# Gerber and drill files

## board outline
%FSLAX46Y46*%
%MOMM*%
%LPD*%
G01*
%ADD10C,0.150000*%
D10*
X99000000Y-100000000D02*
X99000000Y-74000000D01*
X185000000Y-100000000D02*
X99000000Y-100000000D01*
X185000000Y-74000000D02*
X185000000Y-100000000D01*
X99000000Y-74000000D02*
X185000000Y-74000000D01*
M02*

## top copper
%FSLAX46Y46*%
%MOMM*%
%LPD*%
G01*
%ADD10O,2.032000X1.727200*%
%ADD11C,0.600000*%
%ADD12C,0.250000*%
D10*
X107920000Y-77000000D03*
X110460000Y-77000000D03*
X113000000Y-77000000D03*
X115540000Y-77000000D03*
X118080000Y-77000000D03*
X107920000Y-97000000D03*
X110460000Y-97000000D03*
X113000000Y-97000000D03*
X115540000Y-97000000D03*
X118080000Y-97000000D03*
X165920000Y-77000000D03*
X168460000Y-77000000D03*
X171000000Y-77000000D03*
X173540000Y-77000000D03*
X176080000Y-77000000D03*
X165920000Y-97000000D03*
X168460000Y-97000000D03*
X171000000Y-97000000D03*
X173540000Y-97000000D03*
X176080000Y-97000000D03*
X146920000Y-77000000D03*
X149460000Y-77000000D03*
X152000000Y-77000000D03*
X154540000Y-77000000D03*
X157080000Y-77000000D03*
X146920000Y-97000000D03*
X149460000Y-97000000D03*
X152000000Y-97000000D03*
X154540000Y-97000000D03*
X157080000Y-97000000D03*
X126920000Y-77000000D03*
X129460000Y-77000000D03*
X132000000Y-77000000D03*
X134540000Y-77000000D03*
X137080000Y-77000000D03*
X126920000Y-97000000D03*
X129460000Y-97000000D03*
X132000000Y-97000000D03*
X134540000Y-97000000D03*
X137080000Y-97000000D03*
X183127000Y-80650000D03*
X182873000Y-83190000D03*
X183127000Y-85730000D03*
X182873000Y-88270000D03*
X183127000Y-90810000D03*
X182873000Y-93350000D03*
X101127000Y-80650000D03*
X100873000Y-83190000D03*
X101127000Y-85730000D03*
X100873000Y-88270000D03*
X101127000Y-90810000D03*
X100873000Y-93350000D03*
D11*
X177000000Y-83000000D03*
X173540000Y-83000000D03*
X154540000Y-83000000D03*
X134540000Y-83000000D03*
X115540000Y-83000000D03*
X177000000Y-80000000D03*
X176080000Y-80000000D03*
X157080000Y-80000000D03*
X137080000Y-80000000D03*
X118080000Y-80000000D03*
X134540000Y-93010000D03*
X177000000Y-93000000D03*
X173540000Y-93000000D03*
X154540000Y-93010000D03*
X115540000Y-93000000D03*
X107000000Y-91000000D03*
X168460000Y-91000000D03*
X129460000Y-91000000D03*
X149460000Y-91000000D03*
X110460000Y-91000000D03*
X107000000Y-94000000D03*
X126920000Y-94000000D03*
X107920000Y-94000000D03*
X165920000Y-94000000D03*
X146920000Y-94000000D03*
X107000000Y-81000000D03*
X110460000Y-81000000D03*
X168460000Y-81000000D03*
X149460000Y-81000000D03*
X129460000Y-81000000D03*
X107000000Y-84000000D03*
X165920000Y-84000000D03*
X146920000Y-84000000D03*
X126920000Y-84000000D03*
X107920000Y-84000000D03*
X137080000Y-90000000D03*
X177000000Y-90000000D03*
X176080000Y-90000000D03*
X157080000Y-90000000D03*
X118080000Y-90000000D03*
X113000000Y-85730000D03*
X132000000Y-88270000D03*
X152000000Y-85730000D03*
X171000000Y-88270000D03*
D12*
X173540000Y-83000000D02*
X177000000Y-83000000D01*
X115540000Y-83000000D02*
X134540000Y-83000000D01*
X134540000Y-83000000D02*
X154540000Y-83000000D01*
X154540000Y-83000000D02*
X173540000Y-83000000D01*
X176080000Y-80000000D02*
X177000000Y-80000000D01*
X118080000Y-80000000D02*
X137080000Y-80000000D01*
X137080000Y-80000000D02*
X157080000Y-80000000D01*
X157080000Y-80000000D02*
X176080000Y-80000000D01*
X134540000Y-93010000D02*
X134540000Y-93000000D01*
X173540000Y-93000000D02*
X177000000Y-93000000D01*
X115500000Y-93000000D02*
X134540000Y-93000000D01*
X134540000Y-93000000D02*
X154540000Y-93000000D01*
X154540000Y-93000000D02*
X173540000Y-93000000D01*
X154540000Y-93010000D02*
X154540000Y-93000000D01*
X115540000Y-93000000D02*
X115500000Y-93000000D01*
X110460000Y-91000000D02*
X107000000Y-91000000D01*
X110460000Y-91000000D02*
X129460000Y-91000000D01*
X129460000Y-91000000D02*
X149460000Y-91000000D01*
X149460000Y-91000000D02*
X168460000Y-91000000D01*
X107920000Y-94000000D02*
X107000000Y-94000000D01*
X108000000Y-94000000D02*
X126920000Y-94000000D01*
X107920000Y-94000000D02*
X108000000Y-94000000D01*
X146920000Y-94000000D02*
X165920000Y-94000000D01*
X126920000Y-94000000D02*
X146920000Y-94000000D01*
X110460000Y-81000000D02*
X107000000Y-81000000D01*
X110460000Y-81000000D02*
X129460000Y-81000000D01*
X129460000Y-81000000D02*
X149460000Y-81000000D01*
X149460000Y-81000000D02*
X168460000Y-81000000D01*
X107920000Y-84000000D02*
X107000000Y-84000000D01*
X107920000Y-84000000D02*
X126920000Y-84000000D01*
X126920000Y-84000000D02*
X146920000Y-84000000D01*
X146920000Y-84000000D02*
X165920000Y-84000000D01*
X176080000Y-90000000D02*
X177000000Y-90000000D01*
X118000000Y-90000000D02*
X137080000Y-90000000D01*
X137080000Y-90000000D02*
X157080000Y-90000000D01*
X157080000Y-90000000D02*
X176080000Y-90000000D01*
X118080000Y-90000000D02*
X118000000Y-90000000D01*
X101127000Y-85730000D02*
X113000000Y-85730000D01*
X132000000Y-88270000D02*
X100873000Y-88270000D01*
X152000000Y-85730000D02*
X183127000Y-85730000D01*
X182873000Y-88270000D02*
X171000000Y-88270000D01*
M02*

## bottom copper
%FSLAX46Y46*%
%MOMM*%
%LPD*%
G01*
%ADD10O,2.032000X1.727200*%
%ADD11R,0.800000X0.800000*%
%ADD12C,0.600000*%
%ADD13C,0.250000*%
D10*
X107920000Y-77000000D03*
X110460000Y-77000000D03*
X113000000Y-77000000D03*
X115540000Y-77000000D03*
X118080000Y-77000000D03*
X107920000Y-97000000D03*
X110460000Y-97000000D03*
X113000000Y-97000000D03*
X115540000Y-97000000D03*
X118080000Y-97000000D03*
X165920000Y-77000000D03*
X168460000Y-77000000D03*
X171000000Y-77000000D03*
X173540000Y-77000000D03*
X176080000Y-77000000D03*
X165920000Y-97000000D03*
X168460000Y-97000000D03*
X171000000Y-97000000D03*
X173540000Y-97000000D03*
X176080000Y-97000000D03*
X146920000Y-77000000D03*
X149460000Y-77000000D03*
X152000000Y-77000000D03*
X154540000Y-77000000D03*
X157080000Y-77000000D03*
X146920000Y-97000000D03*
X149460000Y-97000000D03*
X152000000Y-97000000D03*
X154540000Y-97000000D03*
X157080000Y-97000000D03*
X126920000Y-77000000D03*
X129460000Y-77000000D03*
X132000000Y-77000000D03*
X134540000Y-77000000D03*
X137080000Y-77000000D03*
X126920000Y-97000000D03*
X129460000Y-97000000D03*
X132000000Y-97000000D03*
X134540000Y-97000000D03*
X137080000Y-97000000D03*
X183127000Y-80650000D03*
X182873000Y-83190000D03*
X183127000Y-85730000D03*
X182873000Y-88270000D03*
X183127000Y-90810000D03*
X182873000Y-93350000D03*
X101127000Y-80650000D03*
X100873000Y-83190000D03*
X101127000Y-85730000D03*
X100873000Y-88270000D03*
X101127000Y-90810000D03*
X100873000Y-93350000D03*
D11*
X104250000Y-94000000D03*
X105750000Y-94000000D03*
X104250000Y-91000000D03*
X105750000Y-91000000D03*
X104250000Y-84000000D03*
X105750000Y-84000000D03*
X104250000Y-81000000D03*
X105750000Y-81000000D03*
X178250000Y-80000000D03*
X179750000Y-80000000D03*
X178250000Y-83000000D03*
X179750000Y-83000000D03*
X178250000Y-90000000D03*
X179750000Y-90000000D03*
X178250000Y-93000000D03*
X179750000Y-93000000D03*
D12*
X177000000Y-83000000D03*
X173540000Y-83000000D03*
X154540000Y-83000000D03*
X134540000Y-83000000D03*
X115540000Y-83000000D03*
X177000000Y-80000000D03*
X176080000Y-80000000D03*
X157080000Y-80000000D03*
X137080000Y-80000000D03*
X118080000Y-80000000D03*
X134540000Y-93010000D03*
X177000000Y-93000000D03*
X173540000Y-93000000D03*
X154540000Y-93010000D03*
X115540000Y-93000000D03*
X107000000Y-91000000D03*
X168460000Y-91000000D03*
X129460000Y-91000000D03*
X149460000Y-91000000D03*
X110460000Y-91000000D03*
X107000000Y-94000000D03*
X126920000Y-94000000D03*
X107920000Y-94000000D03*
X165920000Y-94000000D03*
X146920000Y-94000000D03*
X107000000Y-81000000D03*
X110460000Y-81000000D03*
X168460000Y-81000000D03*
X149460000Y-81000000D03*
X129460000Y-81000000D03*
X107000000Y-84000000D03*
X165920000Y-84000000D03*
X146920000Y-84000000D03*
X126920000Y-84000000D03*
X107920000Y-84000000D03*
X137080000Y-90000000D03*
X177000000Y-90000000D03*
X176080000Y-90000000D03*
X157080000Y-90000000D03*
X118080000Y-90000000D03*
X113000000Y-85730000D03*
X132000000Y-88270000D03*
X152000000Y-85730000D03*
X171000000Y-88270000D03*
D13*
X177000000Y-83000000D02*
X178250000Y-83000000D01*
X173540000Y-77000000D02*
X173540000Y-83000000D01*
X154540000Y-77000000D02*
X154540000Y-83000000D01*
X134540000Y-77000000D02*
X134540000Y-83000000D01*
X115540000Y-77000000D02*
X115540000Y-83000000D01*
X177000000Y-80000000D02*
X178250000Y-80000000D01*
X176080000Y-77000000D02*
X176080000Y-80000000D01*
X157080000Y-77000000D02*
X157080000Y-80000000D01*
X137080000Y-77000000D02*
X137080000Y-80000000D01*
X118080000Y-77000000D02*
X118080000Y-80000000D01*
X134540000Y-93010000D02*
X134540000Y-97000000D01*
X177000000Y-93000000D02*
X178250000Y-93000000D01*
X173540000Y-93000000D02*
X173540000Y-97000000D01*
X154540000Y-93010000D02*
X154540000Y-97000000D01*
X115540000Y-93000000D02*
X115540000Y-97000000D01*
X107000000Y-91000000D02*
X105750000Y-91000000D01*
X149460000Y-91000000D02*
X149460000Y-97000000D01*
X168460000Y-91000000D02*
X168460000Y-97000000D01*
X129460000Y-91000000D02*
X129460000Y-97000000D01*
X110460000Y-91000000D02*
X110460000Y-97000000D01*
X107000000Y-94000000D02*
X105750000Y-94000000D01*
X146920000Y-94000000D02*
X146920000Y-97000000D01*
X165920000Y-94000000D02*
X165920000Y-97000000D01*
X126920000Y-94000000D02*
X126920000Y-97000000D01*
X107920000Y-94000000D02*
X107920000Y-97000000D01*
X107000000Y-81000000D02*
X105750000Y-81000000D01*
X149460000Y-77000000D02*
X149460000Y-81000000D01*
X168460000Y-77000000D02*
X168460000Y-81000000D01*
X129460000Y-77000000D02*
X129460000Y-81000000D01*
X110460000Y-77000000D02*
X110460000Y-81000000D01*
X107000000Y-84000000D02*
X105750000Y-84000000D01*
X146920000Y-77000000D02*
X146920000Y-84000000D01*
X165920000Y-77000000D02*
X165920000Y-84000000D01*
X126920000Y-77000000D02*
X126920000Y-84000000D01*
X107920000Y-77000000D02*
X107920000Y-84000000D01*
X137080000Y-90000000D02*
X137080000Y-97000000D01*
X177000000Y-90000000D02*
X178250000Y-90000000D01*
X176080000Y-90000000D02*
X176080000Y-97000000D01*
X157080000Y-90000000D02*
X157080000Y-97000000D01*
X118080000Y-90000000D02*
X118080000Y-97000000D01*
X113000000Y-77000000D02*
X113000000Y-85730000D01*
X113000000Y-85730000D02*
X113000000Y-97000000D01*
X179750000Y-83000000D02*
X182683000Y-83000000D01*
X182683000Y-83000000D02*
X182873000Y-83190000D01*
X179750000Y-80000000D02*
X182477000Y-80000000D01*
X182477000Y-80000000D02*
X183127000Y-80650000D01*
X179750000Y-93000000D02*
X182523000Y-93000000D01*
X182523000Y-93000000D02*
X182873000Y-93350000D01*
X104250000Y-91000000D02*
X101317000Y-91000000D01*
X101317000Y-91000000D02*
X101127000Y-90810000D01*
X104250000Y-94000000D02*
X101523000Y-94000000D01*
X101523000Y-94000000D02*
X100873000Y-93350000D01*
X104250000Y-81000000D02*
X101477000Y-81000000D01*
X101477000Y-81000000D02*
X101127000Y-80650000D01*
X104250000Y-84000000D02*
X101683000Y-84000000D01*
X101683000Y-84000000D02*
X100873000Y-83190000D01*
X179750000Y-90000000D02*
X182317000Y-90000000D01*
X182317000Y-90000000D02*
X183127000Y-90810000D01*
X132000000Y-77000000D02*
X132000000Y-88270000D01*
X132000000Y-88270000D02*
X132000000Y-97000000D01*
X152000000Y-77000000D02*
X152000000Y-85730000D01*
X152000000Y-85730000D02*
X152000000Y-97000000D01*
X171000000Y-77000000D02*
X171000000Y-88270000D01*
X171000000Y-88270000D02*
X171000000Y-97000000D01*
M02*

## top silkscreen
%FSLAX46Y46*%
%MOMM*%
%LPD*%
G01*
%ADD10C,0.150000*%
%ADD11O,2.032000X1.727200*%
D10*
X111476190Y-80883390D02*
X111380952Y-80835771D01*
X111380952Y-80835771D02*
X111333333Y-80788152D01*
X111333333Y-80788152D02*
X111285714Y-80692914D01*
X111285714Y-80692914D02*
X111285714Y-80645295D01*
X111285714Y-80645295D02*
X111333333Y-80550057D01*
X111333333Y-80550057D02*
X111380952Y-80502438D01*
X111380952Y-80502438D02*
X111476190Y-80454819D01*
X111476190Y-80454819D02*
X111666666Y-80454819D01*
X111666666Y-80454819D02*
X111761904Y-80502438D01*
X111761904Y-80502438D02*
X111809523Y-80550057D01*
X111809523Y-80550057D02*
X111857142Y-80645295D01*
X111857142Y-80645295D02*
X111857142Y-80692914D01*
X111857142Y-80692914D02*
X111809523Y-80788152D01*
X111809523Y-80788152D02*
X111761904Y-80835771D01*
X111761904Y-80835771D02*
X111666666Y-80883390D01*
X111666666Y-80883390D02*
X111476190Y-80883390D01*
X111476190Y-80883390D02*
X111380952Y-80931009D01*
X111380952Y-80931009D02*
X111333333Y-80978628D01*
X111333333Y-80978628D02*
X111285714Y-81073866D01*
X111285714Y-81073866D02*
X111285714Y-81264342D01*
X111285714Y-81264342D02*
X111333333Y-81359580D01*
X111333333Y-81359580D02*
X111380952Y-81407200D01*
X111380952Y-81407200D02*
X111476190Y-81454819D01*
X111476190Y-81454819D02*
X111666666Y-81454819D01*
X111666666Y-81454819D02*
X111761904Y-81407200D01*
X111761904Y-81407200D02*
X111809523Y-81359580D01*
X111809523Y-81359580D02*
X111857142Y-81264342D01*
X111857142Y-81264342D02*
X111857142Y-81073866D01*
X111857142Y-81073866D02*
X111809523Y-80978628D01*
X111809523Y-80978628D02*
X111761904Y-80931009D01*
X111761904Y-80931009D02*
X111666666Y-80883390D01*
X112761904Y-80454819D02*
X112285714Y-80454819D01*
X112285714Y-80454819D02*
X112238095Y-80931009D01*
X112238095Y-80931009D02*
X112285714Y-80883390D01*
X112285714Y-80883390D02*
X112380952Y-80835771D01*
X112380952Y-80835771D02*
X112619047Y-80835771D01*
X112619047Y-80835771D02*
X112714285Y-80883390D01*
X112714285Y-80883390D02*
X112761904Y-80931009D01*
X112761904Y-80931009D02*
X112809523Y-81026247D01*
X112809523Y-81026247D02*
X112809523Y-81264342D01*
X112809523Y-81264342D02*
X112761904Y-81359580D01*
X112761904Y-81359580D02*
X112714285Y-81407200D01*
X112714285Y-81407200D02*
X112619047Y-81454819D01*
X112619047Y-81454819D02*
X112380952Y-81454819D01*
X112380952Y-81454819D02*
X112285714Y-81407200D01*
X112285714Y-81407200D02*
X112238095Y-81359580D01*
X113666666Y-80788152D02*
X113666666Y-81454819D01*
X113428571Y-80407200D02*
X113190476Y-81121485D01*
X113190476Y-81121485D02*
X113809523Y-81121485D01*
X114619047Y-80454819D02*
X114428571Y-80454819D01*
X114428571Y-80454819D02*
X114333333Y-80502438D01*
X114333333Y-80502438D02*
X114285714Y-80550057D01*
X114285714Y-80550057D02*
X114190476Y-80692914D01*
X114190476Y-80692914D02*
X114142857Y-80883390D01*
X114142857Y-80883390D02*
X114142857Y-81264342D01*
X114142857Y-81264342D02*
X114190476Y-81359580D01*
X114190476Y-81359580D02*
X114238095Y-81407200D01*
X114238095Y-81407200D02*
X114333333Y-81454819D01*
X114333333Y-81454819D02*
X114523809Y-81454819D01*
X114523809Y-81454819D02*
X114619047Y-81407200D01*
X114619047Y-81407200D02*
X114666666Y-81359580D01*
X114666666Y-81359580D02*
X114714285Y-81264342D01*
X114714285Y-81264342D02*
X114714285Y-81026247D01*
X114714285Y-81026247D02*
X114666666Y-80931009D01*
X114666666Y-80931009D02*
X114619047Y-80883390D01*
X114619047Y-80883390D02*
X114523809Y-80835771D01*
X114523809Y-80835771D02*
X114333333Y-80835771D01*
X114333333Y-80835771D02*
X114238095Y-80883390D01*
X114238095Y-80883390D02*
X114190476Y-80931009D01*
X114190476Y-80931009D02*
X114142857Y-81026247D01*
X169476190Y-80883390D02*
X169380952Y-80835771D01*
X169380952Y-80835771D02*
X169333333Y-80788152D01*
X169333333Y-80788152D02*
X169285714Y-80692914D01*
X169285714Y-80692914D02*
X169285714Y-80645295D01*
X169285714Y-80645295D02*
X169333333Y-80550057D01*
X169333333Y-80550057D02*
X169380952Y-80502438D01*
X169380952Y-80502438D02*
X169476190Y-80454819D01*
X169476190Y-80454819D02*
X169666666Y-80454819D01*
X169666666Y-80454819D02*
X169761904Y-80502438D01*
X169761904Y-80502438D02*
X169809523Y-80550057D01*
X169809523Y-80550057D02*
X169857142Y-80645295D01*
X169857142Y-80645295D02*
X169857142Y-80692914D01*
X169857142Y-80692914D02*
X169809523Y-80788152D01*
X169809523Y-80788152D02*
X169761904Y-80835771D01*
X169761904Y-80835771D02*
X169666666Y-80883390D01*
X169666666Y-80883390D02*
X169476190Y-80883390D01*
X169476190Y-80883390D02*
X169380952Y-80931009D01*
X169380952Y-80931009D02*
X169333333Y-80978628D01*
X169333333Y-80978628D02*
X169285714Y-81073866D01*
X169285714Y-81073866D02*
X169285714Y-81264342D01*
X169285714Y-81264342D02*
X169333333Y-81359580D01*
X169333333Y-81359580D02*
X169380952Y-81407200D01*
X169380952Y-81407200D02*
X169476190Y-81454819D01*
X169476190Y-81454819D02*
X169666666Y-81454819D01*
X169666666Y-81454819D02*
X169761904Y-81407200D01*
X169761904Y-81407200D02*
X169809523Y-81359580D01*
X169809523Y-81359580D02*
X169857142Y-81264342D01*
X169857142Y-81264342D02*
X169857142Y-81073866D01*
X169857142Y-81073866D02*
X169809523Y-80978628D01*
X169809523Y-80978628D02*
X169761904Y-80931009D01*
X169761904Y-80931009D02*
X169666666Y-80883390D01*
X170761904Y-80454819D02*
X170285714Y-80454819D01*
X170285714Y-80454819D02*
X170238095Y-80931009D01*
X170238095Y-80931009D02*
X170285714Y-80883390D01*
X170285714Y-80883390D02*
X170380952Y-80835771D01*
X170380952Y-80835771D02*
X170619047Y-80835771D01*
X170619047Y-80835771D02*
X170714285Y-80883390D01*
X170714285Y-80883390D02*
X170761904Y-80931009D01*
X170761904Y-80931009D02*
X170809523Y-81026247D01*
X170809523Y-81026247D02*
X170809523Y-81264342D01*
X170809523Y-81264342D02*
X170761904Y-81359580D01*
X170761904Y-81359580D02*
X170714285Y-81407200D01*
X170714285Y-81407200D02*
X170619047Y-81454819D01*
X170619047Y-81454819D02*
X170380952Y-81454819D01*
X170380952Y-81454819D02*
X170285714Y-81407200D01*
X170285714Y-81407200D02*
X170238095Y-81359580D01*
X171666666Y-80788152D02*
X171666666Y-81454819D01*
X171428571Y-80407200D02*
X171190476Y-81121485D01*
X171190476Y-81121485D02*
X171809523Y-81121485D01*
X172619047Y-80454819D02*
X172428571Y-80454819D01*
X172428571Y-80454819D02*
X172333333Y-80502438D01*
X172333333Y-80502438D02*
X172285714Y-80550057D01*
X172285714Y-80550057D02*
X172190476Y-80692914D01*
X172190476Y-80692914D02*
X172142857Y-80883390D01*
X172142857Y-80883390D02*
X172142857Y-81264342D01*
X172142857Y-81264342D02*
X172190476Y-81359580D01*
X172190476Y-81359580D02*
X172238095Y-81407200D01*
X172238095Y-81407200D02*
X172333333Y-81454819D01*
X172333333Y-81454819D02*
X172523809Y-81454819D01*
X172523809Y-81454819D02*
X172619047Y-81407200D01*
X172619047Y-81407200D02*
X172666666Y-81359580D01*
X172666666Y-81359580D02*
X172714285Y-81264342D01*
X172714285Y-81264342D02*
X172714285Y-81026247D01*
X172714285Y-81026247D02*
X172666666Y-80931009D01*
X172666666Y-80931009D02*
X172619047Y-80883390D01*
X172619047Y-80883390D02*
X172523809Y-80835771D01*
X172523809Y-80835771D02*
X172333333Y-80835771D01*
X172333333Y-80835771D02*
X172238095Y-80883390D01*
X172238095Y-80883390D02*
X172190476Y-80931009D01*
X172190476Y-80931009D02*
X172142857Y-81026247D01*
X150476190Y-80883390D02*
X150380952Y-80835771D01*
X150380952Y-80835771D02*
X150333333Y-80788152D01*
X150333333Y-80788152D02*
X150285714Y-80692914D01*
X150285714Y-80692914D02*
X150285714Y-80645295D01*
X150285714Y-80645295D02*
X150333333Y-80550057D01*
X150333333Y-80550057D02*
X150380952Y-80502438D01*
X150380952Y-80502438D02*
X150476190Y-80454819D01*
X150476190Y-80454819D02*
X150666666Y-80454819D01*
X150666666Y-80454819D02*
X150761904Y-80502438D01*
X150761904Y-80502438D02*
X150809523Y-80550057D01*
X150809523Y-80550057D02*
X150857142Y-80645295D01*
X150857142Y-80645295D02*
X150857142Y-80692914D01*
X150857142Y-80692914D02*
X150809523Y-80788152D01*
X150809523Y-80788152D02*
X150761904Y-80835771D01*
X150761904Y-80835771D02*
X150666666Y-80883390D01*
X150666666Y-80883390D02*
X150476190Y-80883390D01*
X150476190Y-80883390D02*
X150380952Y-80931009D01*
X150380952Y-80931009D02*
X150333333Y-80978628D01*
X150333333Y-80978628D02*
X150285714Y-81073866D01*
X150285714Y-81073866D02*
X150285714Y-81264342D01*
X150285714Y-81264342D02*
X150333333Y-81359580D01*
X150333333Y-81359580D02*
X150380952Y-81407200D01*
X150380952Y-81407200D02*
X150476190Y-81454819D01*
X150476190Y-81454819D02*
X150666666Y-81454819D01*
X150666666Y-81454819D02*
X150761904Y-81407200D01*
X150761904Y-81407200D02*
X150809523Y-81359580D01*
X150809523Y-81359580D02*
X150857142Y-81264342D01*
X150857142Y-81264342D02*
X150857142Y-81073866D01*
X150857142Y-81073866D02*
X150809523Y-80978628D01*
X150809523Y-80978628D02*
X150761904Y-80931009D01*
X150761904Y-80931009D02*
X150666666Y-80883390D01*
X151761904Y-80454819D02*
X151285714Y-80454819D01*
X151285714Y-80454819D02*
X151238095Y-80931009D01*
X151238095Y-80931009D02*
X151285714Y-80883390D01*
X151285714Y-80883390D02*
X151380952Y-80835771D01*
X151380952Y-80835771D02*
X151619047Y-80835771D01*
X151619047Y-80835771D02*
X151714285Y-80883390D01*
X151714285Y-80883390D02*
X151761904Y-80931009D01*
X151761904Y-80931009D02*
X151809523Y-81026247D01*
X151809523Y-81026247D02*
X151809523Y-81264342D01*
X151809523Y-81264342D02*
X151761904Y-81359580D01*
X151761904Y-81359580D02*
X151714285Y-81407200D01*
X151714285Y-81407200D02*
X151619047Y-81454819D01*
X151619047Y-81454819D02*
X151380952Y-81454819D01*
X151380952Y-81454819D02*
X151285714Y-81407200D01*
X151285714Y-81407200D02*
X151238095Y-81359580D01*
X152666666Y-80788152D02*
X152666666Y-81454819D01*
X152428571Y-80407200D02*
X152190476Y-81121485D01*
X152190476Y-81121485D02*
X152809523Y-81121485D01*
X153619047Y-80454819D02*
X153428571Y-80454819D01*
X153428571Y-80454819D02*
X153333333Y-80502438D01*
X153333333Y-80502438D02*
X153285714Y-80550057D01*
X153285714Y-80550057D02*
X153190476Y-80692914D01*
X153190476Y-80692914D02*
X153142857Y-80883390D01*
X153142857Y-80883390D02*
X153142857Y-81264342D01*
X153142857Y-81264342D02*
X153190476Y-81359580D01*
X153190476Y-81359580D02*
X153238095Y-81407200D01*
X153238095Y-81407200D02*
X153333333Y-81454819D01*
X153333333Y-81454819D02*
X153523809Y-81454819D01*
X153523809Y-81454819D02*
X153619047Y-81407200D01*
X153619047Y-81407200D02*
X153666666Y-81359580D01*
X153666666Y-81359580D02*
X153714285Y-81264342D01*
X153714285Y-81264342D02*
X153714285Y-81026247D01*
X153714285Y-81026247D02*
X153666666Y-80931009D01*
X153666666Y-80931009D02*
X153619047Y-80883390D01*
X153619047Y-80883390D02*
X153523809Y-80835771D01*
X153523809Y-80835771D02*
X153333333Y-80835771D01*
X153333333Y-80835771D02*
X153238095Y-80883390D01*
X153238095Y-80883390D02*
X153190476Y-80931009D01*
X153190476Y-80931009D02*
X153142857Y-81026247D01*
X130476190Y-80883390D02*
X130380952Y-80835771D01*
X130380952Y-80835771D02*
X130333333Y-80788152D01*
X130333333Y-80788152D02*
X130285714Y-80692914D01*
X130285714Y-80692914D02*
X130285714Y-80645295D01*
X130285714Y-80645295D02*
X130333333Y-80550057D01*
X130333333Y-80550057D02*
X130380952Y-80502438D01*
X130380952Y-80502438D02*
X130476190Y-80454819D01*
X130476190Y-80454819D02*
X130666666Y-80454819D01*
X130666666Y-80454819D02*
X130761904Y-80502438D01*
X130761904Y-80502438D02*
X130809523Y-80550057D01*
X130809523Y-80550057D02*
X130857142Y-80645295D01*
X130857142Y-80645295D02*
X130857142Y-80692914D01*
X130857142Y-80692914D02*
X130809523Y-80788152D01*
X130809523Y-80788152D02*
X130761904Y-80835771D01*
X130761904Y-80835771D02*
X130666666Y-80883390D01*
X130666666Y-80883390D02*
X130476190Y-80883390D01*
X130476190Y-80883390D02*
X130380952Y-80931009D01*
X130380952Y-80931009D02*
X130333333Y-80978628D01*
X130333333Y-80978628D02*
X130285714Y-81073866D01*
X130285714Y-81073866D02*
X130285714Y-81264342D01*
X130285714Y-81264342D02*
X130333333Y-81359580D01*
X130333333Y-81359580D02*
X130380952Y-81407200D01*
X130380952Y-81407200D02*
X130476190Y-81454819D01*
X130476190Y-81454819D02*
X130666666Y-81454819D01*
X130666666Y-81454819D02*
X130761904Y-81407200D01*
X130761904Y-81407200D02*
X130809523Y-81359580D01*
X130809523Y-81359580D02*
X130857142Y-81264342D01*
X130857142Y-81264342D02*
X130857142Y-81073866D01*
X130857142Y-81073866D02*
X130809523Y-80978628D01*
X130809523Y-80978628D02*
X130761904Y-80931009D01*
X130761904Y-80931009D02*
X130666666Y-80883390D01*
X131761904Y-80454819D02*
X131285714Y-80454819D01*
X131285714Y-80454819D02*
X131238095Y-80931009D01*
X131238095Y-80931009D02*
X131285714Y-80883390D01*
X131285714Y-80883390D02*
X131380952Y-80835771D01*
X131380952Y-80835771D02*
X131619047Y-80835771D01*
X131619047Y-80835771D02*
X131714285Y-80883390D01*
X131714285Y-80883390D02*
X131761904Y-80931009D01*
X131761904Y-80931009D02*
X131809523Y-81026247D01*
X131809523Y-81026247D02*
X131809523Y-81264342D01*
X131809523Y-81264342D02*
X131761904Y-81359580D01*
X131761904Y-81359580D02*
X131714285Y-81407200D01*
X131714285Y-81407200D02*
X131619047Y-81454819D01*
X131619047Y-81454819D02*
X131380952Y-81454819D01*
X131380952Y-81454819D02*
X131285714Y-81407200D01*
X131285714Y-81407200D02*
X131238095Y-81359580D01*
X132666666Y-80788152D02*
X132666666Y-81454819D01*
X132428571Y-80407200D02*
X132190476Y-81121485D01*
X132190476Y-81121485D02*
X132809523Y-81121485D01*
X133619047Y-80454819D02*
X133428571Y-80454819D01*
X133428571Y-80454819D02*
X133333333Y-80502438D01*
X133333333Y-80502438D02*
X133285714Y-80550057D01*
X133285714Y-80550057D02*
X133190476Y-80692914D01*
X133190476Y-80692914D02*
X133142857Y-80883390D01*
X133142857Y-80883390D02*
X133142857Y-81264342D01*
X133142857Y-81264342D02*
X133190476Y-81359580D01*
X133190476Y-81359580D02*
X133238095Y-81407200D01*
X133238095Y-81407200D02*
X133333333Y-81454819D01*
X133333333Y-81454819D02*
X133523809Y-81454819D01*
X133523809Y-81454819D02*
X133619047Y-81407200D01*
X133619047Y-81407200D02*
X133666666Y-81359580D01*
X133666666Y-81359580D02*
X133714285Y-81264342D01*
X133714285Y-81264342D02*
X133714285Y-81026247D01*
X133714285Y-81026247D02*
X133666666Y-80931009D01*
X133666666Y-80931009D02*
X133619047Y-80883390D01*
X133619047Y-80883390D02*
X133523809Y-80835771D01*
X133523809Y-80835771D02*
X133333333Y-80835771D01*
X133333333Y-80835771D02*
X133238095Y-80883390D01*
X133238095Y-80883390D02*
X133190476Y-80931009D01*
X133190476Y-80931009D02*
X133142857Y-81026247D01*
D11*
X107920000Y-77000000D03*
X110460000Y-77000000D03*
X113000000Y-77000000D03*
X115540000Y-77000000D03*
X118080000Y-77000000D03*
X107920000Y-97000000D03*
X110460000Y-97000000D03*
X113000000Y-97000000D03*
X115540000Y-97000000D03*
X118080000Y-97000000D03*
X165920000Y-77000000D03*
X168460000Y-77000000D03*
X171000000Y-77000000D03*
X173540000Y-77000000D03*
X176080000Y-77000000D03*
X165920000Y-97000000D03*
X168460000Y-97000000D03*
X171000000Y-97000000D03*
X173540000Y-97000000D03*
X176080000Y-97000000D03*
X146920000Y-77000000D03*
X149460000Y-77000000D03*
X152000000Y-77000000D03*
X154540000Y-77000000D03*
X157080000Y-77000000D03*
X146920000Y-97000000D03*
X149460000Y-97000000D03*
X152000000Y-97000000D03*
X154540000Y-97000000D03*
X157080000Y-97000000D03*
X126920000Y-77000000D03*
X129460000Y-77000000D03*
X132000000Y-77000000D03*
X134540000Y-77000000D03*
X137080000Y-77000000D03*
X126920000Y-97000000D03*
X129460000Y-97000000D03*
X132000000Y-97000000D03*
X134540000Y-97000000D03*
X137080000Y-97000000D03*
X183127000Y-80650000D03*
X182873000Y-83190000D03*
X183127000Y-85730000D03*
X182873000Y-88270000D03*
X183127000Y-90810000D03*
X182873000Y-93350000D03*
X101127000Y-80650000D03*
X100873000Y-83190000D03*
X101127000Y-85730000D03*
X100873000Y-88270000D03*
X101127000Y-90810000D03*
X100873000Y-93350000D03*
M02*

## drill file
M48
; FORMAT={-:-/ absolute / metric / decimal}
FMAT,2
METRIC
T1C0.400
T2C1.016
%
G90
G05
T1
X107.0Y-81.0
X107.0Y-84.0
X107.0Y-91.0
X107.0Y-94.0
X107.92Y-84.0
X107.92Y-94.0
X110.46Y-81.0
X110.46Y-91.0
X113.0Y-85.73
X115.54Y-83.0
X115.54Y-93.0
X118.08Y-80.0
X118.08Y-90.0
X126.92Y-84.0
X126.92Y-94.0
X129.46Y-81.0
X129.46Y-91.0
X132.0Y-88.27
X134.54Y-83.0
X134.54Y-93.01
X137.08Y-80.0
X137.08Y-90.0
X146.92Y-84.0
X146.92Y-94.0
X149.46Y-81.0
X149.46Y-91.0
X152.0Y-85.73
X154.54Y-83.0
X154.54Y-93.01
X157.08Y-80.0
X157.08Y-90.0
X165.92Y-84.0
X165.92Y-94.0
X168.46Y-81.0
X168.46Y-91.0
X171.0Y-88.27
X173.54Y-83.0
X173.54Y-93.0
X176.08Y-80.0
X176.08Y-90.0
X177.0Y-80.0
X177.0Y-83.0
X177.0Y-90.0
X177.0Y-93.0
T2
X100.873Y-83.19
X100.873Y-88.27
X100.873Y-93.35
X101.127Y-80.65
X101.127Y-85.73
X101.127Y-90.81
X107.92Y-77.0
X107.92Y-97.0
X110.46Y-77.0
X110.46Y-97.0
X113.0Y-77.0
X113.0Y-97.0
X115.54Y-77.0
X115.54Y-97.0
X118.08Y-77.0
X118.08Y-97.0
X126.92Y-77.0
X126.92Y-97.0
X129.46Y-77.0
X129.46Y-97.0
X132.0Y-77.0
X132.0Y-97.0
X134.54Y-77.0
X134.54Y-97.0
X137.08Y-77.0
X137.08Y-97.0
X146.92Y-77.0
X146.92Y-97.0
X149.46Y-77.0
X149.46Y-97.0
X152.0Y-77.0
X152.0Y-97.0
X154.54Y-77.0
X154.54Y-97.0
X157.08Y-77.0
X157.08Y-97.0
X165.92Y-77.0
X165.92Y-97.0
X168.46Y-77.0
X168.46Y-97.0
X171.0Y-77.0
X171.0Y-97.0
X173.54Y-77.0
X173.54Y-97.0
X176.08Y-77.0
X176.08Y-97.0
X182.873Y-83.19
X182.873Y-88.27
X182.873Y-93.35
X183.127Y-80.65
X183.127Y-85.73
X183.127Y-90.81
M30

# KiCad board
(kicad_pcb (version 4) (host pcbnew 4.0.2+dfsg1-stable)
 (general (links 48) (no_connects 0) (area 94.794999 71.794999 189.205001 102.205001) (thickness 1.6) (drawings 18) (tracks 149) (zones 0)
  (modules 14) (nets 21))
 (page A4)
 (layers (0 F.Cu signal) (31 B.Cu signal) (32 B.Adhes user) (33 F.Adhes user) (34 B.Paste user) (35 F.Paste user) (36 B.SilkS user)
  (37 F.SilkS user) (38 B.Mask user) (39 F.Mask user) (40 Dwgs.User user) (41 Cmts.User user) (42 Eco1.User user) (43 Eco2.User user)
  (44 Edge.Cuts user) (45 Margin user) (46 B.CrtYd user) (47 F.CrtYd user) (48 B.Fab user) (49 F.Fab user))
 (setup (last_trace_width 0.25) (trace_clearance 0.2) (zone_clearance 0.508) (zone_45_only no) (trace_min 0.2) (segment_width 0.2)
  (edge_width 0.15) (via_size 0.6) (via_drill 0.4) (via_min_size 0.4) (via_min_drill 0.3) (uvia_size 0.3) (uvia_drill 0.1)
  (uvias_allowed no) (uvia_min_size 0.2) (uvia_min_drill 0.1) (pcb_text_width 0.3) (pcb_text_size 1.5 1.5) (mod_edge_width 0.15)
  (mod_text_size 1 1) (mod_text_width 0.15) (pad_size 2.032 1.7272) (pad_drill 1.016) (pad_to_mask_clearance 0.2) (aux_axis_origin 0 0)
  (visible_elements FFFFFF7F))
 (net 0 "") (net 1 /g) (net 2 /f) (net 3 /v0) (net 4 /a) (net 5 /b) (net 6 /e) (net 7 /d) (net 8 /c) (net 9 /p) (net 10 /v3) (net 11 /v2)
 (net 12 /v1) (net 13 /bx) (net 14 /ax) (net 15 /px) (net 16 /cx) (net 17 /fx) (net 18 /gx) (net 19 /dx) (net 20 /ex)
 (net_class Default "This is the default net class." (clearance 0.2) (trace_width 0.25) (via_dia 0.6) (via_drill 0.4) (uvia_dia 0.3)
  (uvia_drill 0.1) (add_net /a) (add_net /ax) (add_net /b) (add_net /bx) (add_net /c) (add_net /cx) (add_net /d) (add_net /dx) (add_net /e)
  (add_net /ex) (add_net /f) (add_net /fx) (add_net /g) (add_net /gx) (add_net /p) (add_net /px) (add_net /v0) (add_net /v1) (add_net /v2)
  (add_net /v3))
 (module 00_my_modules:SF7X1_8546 (layer F.Cu) (at 113 87)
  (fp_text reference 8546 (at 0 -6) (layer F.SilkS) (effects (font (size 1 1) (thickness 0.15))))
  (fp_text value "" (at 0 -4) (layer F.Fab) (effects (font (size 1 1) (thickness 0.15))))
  (pad G thru_hole oval (at -5.08 -10) (size 2.032 1.7272) (drill 1.016) (layers *.Cu *.Mask F.SilkS) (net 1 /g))
  (pad F thru_hole oval (at -2.54 -10) (size 2.032 1.7272) (drill 1.016) (layers *.Cu *.Mask F.SilkS) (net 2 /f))
  (pad V thru_hole oval (at 0 -10) (size 2.032 1.7272) (drill 1.016) (layers *.Cu *.Mask F.SilkS) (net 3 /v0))
  (pad A thru_hole oval (at 2.54 -10) (size 2.032 1.7272) (drill 1.016) (layers *.Cu *.Mask F.SilkS) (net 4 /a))
  (pad B thru_hole oval (at 5.08 -10) (size 2.032 1.7272) (drill 1.016) (layers *.Cu *.Mask F.SilkS) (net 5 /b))
  (pad E thru_hole oval (at -5.08 10) (size 2.032 1.7272) (drill 1.016) (layers *.Cu *.Mask F.SilkS) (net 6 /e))
  (pad D thru_hole oval (at -2.54 10) (size 2.032 1.7272) (drill 1.016) (layers *.Cu *.Mask F.SilkS) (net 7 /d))
  (pad V thru_hole oval (at 0 10) (size 2.032 1.7272) (drill 1.016) (layers *.Cu *.Mask F.SilkS) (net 3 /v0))
  (pad C thru_hole oval (at 2.54 10) (size 2.032 1.7272) (drill 1.016) (layers *.Cu *.Mask F.SilkS) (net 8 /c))
  (pad P thru_hole oval (at 5.08 10) (size 2.032 1.7272) (drill 1.016) (layers *.Cu *.Mask F.SilkS) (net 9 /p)))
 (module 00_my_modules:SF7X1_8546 (layer F.Cu) (at 171 87)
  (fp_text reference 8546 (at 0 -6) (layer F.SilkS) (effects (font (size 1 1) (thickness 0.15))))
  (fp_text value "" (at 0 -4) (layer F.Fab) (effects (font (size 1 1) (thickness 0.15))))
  (pad G thru_hole oval (at -5.08 -10) (size 2.032 1.7272) (drill 1.016) (layers *.Cu *.Mask F.SilkS) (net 1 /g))
  (pad F thru_hole oval (at -2.54 -10) (size 2.032 1.7272) (drill 1.016) (layers *.Cu *.Mask F.SilkS) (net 2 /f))
  (pad V thru_hole oval (at 0 -10) (size 2.032 1.7272) (drill 1.016) (layers *.Cu *.Mask F.SilkS) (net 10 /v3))
  (pad A thru_hole oval (at 2.54 -10) (size 2.032 1.7272) (drill 1.016) (layers *.Cu *.Mask F.SilkS) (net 4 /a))
  (pad B thru_hole oval (at 5.08 -10) (size 2.032 1.7272) (drill 1.016) (layers *.Cu *.Mask F.SilkS) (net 5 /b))
  (pad E thru_hole oval (at -5.08 10) (size 2.032 1.7272) (drill 1.016) (layers *.Cu *.Mask F.SilkS) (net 6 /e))
  (pad D thru_hole oval (at -2.54 10) (size 2.032 1.7272) (drill 1.016) (layers *.Cu *.Mask F.SilkS) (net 7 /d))
  (pad V thru_hole oval (at 0 10) (size 2.032 1.7272) (drill 1.016) (layers *.Cu *.Mask F.SilkS) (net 10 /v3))
  (pad C thru_hole oval (at 2.54 10) (size 2.032 1.7272) (drill 1.016) (layers *.Cu *.Mask F.SilkS) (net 8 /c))
  (pad P thru_hole oval (at 5.08 10) (size 2.032 1.7272) (drill 1.016) (layers *.Cu *.Mask F.SilkS) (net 9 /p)))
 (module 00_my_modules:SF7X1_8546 (layer F.Cu) (at 152 87)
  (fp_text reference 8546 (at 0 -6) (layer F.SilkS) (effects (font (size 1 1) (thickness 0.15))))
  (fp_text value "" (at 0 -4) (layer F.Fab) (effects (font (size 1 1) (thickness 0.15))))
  (pad G thru_hole oval (at -5.08 -10) (size 2.032 1.7272) (drill 1.016) (layers *.Cu *.Mask F.SilkS) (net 1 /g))
  (pad F thru_hole oval (at -2.54 -10) (size 2.032 1.7272) (drill 1.016) (layers *.Cu *.Mask F.SilkS) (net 2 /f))
  (pad V thru_hole oval (at 0 -10) (size 2.032 1.7272) (drill 1.016) (layers *.Cu *.Mask F.SilkS) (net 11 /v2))
  (pad A thru_hole oval (at 2.54 -10) (size 2.032 1.7272) (drill 1.016) (layers *.Cu *.Mask F.SilkS) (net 4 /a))
  (pad B thru_hole oval (at 5.08 -10) (size 2.032 1.7272) (drill 1.016) (layers *.Cu *.Mask F.SilkS) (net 5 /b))
  (pad E thru_hole oval (at -5.08 10) (size 2.032 1.7272) (drill 1.016) (layers *.Cu *.Mask F.SilkS) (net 6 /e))
  (pad D thru_hole oval (at -2.54 10) (size 2.032 1.7272) (drill 1.016) (layers *.Cu *.Mask F.SilkS) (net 7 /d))
  (pad V thru_hole oval (at 0 10) (size 2.032 1.7272) (drill 1.016) (layers *.Cu *.Mask F.SilkS) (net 11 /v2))
  (pad C thru_hole oval (at 2.54 10) (size 2.032 1.7272) (drill 1.016) (layers *.Cu *.Mask F.SilkS) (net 8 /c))
  (pad P thru_hole oval (at 5.08 10) (size 2.032 1.7272) (drill 1.016) (layers *.Cu *.Mask F.SilkS) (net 9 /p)))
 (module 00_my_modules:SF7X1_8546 (layer F.Cu) (at 132 87)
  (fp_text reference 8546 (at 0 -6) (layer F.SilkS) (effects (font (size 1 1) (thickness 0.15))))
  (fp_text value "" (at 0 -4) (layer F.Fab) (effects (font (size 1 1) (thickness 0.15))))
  (pad G thru_hole oval (at -5.08 -10) (size 2.032 1.7272) (drill 1.016) (layers *.Cu *.Mask F.SilkS) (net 1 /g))
  (pad F thru_hole oval (at -2.54 -10) (size 2.032 1.7272) (drill 1.016) (layers *.Cu *.Mask F.SilkS) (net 2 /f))
  (pad V thru_hole oval (at 0 -10) (size 2.032 1.7272) (drill 1.016) (layers *.Cu *.Mask F.SilkS) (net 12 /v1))
  (pad A thru_hole oval (at 2.54 -10) (size 2.032 1.7272) (drill 1.016) (layers *.Cu *.Mask F.SilkS) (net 4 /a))
  (pad B thru_hole oval (at 5.08 -10) (size 2.032 1.7272) (drill 1.016) (layers *.Cu *.Mask F.SilkS) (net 5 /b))
  (pad E thru_hole oval (at -5.08 10) (size 2.032 1.7272) (drill 1.016) (layers *.Cu *.Mask F.SilkS) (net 6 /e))
  (pad D thru_hole oval (at -2.54 10) (size 2.032 1.7272) (drill 1.016) (layers *.Cu *.Mask F.SilkS) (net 7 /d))
  (pad V thru_hole oval (at 0 10) (size 2.032 1.7272) (drill 1.016) (layers *.Cu *.Mask F.SilkS) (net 12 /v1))
  (pad C thru_hole oval (at 2.54 10) (size 2.032 1.7272) (drill 1.016) (layers *.Cu *.Mask F.SilkS) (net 8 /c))
  (pad P thru_hole oval (at 5.08 10) (size 2.032 1.7272) (drill 1.016) (layers *.Cu *.Mask F.SilkS) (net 9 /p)))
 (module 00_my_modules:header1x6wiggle (layer F.Cu) (at 183 87)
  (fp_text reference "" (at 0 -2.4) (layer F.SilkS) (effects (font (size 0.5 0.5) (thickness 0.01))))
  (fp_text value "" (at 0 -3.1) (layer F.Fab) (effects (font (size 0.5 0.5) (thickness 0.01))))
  (pad 1 thru_hole oval (at 0.127 -6.35) (size 2.032 1.7272) (drill 1.016) (layers *.Cu *.Mask F.SilkS) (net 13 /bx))
  (pad 2 thru_hole oval (at -0.127 -3.81) (size 2.032 1.7272) (drill 1.016) (layers *.Cu *.Mask F.SilkS) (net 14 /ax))
  (pad 3 thru_hole oval (at 0.127 -1.27) (size 2.032 1.7272) (drill 1.016) (layers *.Cu *.Mask F.SilkS) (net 11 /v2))
  (pad 4 thru_hole oval (at -0.127 1.27) (size 2.032 1.7272) (drill 1.016) (layers *.Cu *.Mask F.SilkS) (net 10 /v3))
  (pad 5 thru_hole oval (at 0.127 3.81) (size 2.032 1.7272) (drill 1.016) (layers *.Cu *.Mask F.SilkS) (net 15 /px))
  (pad 6 thru_hole oval (at -0.127 6.35) (size 2.032 1.7272) (drill 1.016) (layers *.Cu *.Mask F.SilkS) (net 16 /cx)))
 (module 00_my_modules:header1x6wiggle (layer F.Cu) (at 101 87)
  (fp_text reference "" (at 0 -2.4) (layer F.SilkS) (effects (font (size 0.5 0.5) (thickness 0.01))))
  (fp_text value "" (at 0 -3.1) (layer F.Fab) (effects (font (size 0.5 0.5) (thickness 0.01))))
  (pad 1 thru_hole oval (at 0.127 -6.35) (size 2.032 1.7272) (drill 1.016) (layers *.Cu *.Mask F.SilkS) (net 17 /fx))
  (pad 2 thru_hole oval (at -0.127 -3.81) (size 2.032 1.7272) (drill 1.016) (layers *.Cu *.Mask F.SilkS) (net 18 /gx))
  (pad 3 thru_hole oval (at 0.127 -1.27) (size 2.032 1.7272) (drill 1.016) (layers *.Cu *.Mask F.SilkS) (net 3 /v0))
  (pad 4 thru_hole oval (at -0.127 1.27) (size 2.032 1.7272) (drill 1.016) (layers *.Cu *.Mask F.SilkS) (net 12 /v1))
  (pad 5 thru_hole oval (at 0.127 3.81) (size 2.032 1.7272) (drill 1.016) (layers *.Cu *.Mask F.SilkS) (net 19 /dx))
  (pad 6 thru_hole oval (at -0.127 6.35) (size 2.032 1.7272) (drill 1.016) (layers *.Cu *.Mask F.SilkS) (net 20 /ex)))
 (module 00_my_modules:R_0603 (layer B.Cu) (at 105 94)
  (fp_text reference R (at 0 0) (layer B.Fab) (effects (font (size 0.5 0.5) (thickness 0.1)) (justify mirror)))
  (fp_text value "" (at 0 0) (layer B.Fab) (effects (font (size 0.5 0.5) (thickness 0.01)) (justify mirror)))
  (pad 1 smd rect (at -0.75 0) (size 0.8 0.8) (layers B.Cu B.Paste B.Mask) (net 20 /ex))
  (pad 2 smd rect (at 0.75 0) (size 0.8 0.8) (layers B.Cu B.Paste B.Mask) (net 6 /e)))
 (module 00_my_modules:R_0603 (layer B.Cu) (at 105 91)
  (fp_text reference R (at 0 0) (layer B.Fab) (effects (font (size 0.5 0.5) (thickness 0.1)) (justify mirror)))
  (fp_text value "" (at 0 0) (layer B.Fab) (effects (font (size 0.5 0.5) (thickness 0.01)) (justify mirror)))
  (pad 1 smd rect (at -0.75 0) (size 0.8 0.8) (layers B.Cu B.Paste B.Mask) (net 19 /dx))
  (pad 2 smd rect (at 0.75 0) (size 0.8 0.8) (layers B.Cu B.Paste B.Mask) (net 7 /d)))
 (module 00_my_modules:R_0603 (layer B.Cu) (at 105 84)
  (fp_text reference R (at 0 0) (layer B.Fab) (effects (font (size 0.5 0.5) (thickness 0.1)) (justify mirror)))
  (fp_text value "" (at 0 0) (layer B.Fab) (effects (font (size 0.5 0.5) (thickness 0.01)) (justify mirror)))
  (pad 1 smd rect (at -0.75 0) (size 0.8 0.8) (layers B.Cu B.Paste B.Mask) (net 18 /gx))
  (pad 2 smd rect (at 0.75 0) (size 0.8 0.8) (layers B.Cu B.Paste B.Mask) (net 1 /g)))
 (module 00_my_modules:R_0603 (layer B.Cu) (at 105 81)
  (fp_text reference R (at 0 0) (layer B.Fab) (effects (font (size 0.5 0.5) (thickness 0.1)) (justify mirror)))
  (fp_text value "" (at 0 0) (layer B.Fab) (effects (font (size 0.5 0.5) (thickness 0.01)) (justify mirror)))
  (pad 1 smd rect (at -0.75 0) (size 0.8 0.8) (layers B.Cu B.Paste B.Mask) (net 17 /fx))
  (pad 2 smd rect (at 0.75 0) (size 0.8 0.8) (layers B.Cu B.Paste B.Mask) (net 2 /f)))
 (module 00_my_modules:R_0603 (layer B.Cu) (at 179 80)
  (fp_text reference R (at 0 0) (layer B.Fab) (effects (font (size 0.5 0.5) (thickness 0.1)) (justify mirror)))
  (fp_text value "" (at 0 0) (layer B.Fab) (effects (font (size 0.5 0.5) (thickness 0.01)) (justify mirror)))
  (pad 1 smd rect (at -0.75 0) (size 0.8 0.8) (layers B.Cu B.Paste B.Mask) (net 5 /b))
  (pad 2 smd rect (at 0.75 0) (size 0.8 0.8) (layers B.Cu B.Paste B.Mask) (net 13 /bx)))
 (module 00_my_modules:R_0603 (layer B.Cu) (at 179 83)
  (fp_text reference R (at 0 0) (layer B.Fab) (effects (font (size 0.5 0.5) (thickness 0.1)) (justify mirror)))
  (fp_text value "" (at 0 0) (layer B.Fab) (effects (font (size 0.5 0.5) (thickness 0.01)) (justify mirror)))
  (pad 1 smd rect (at -0.75 0) (size 0.8 0.8) (layers B.Cu B.Paste B.Mask) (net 4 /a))
  (pad 2 smd rect (at 0.75 0) (size 0.8 0.8) (layers B.Cu B.Paste B.Mask) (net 14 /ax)))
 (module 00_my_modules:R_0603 (layer B.Cu) (at 179 90)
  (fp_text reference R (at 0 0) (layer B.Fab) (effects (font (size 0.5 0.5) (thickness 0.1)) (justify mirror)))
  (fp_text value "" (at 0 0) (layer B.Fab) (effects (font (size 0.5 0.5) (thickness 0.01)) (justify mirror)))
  (pad 1 smd rect (at -0.75 0) (size 0.8 0.8) (layers B.Cu B.Paste B.Mask) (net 9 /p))
  (pad 2 smd rect (at 0.75 0) (size 0.8 0.8) (layers B.Cu B.Paste B.Mask) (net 15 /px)))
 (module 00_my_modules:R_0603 (layer B.Cu) (at 179 93)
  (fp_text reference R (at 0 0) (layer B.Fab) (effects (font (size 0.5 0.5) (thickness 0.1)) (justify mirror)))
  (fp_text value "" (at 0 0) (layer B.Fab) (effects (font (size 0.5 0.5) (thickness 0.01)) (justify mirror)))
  (pad 1 smd rect (at -0.75 0) (size 0.8 0.8) (layers B.Cu B.Paste B.Mask) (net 8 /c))
  (pad 2 smd rect (at 0.75 0) (size 0.8 0.8) (layers B.Cu B.Paste B.Mask) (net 16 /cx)))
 (gr_line (start 99 100) (end 99 74) (angle 90) (layer Edge.Cuts) (width 0.15))
 (gr_line (start 185 100) (end 99 100) (angle 90) (layer Edge.Cuts) (width 0.15))
 (gr_line (start 185 74) (end 185 100) (angle 90) (layer Edge.Cuts) (width 0.15))
 (gr_line (start 99 74) (end 185 74) (angle 90) (layer Edge.Cuts) (width 0.15))
 (segment (start 173.54 83) (end 177 83) (width 0.25) (layer F.Cu) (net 4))
 (segment (start 177 83) (end 178.25 83) (width 0.25) (layer B.Cu) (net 4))
 (via (at 177 83) (size 0.6) (drill 0.4) (layers F.Cu B.Cu) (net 4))
 (segment (start 115.54 83) (end 134.54 83) (width 0.25) (layer F.Cu) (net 4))
 (segment (start 134.54 83) (end 154.54 83) (width 0.25) (layer F.Cu) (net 4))
 (segment (start 154.54 83) (end 173.54 83) (width 0.25) (layer F.Cu) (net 4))
 (via (at 173.54 83) (size 0.6) (drill 0.4) (layers F.Cu B.Cu) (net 4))
 (via (at 154.54 83) (size 0.6) (drill 0.4) (layers F.Cu B.Cu) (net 4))
 (via (at 134.54 83) (size 0.6) (drill 0.4) (layers F.Cu B.Cu) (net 4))
 (via (at 115.54 83) (size 0.6) (drill 0.4) (layers F.Cu B.Cu) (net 4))
 (segment (start 173.54 77) (end 173.54 83) (width 0.25) (layer B.Cu) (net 4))
 (segment (start 154.54 77) (end 154.54 83) (width 0.25) (layer B.Cu) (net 4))
 (segment (start 134.54 77) (end 134.54 83) (width 0.25) (layer B.Cu) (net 4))
 (segment (start 115.54 77) (end 115.54 83) (width 0.25) (layer B.Cu) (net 4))
 (segment (start 176.08 80) (end 177 80) (width 0.25) (layer F.Cu) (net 5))
 (segment (start 177 80) (end 178.25 80) (width 0.25) (layer B.Cu) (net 5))
 (via (at 177 80) (size 0.6) (drill 0.4) (layers F.Cu B.Cu) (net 5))
 (segment (start 118.08 80) (end 137.08 80) (width 0.25) (layer F.Cu) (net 5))
 (segment (start 137.08 80) (end 157.08 80) (width 0.25) (layer F.Cu) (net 5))
 (segment (start 157.08 80) (end 176.08 80) (width 0.25) (layer F.Cu) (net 5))
 (via (at 176.08 80) (size 0.6) (drill 0.4) (layers F.Cu B.Cu) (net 5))
 (via (at 157.08 80) (size 0.6) (drill 0.4) (layers F.Cu B.Cu) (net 5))
 (via (at 137.08 80) (size 0.6) (drill 0.4) (layers F.Cu B.Cu) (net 5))
 (via (at 118.08 80) (size 0.6) (drill 0.4) (layers F.Cu B.Cu) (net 5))
 (segment (start 176.08 77) (end 176.08 80) (width 0.25) (layer B.Cu) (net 5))
 (segment (start 157.08 77) (end 157.08 80) (width 0.25) (layer B.Cu) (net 5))
 (segment (start 137.08 77) (end 137.08 80) (width 0.25) (layer B.Cu) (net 5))
 (segment (start 118.08 77) (end 118.08 80) (width 0.25) (layer B.Cu) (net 5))
 (via (at 134.54 93.01) (size 0.6) (drill 0.4) (layers F.Cu B.Cu) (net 8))
 (segment (start 134.54 93.01) (end 134.54 93) (width 0.25) (layer F.Cu) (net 8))
 (segment (start 134.54 93.01) (end 134.54 97) (width 0.25) (layer B.Cu) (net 8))
 (segment (start 173.54 93) (end 177 93) (width 0.25) (layer F.Cu) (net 8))
 (segment (start 177 93) (end 178.25 93) (width 0.25) (layer B.Cu) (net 8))
 (via (at 177 93) (size 0.6) (drill 0.4) (layers F.Cu B.Cu) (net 8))
 (segment (start 115.5 93) (end 134.54 93) (width 0.25) (layer F.Cu) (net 8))
 (segment (start 134.54 93) (end 154.54 93) (width 0.25) (layer F.Cu) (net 8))
 (segment (start 154.54 93) (end 173.54 93) (width 0.25) (layer F.Cu) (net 8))
 (via (at 173.54 93) (size 0.6) (drill 0.4) (layers F.Cu B.Cu) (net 8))
 (via (at 154.54 93.01) (size 0.6) (drill 0.4) (layers F.Cu B.Cu) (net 8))
 (segment (start 154.54 93.01) (end 154.54 93) (width 0.25) (layer F.Cu) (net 8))
 (via (at 115.54 93) (size 0.6) (drill 0.4) (layers F.Cu B.Cu) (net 8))
 (segment (start 115.54 93) (end 115.5 93) (width 0.25) (layer F.Cu) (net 8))
 (segment (start 173.54 93) (end 173.54 97) (width 0.25) (layer B.Cu) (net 8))
 (segment (start 154.54 93.01) (end 154.54 97) (width 0.25) (layer B.Cu) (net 8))
 (segment (start 115.54 93) (end 115.54 97) (width 0.25) (layer B.Cu) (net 8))
 (segment (start 110.46 91) (end 107 91) (width 0.25) (layer F.Cu) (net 7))
 (segment (start 107 91) (end 105.75 91) (width 0.25) (layer B.Cu) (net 7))
 (via (at 107 91) (size 0.6) (drill 0.4) (layers F.Cu B.Cu) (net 7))
 (segment (start 149.46 91) (end 149.46 97) (width 0.25) (layer B.Cu) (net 7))
 (segment (start 168.46 91) (end 168.46 97) (width 0.25) (layer B.Cu) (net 7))
 (segment (start 129.46 91) (end 129.46 97) (width 0.25) (layer B.Cu) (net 7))
 (segment (start 110.46 91) (end 110.46 97) (width 0.25) (layer B.Cu) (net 7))
 (via (at 168.46 91) (size 0.6) (drill 0.4) (layers F.Cu B.Cu) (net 7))
 (via (at 129.46 91) (size 0.6) (drill 0.4) (layers F.Cu B.Cu) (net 7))
 (segment (start 110.46 91) (end 129.46 91) (width 0.25) (layer F.Cu) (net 7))
 (segment (start 129.46 91) (end 149.46 91) (width 0.25) (layer F.Cu) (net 7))
 (segment (start 149.46 91) (end 168.46 91) (width 0.25) (layer F.Cu) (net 7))
 (via (at 149.46 91) (size 0.6) (drill 0.4) (layers F.Cu B.Cu) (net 7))
 (via (at 110.46 91) (size 0.6) (drill 0.4) (layers F.Cu B.Cu) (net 7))
 (segment (start 107.92 94) (end 107 94) (width 0.25) (layer F.Cu) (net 6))
 (segment (start 107 94) (end 105.75 94) (width 0.25) (layer B.Cu) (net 6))
 (via (at 107 94) (size 0.6) (drill 0.4) (layers F.Cu B.Cu) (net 6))
 (segment (start 146.92 94) (end 146.92 97) (width 0.25) (layer B.Cu) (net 6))
 (segment (start 165.92 94) (end 165.92 97) (width 0.25) (layer B.Cu) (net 6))
 (segment (start 126.92 94) (end 126.92 97) (width 0.25) (layer B.Cu) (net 6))
 (segment (start 107.92 94) (end 107.92 97) (width 0.25) (layer B.Cu) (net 6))
 (via (at 126.92 94) (size 0.6) (drill 0.4) (layers F.Cu B.Cu) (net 6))
 (segment (start 108 94) (end 126.92 94) (width 0.25) (layer F.Cu) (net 6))
 (via (at 107.92 94) (size 0.6) (drill 0.4) (layers F.Cu B.Cu) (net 6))
 (segment (start 107.92 94) (end 108 94) (width 0.25) (layer F.Cu) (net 6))
 (via (at 165.92 94) (size 0.6) (drill 0.4) (layers F.Cu B.Cu) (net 6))
 (segment (start 146.92 94) (end 165.92 94) (width 0.25) (layer F.Cu) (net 6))
 (segment (start 126.92 94) (end 146.92 94) (width 0.25) (layer F.Cu) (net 6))
 (via (at 146.92 94) (size 0.6) (drill 0.4) (layers F.Cu B.Cu) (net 6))
 (via (at 107 81) (size 0.6) (drill 0.4) (layers F.Cu B.Cu) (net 2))
 (segment (start 110.46 81) (end 107 81) (width 0.25) (layer F.Cu) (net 2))
 (segment (start 107 81) (end 105.75 81) (width 0.25) (layer B.Cu) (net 2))
 (via (at 110.46 81) (size 0.6) (drill 0.4) (layers F.Cu B.Cu) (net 2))
 (segment (start 110.46 81) (end 129.46 81) (width 0.25) (layer F.Cu) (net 2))
 (segment (start 129.46 81) (end 149.46 81) (width 0.25) (layer F.Cu) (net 2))
 (segment (start 149.46 81) (end 168.46 81) (width 0.25) (layer F.Cu) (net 2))
 (via (at 168.46 81) (size 0.6) (drill 0.4) (layers F.Cu B.Cu) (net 2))
 (via (at 149.46 81) (size 0.6) (drill 0.4) (layers F.Cu B.Cu) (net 2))
 (via (at 129.46 81) (size 0.6) (drill 0.4) (layers F.Cu B.Cu) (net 2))
 (segment (start 149.46 77) (end 149.46 81) (width 0.25) (layer B.Cu) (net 2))
 (segment (start 168.46 77) (end 168.46 81) (width 0.25) (layer B.Cu) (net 2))
 (segment (start 129.46 77) (end 129.46 81) (width 0.25) (layer B.Cu) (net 2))
 (segment (start 110.46 77) (end 110.46 81) (width 0.25) (layer B.Cu) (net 2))
 (via (at 107 84) (size 0.6) (drill 0.4) (layers F.Cu B.Cu) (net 1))
 (segment (start 107.92 84) (end 107 84) (width 0.25) (layer F.Cu) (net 1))
 (segment (start 107 84) (end 105.75 84) (width 0.25) (layer B.Cu) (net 1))
 (segment (start 107.92 84) (end 126.92 84) (width 0.25) (layer F.Cu) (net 1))
 (segment (start 126.92 84) (end 146.92 84) (width 0.25) (layer F.Cu) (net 1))
 (segment (start 146.92 84) (end 165.92 84) (width 0.25) (layer F.Cu) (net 1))
 (via (at 165.92 84) (size 0.6) (drill 0.4) (layers F.Cu B.Cu) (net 1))
 (via (at 146.92 84) (size 0.6) (drill 0.4) (layers F.Cu B.Cu) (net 1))
 (via (at 126.92 84) (size 0.6) (drill 0.4) (layers F.Cu B.Cu) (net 1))
 (via (at 107.92 84) (size 0.6) (drill 0.4) (layers F.Cu B.Cu) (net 1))
 (segment (start 146.92 77) (end 146.92 84) (width 0.25) (layer B.Cu) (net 1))
 (segment (start 165.92 77) (end 165.92 84) (width 0.25) (layer B.Cu) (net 1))
 (segment (start 126.92 77) (end 126.92 84) (width 0.25) (layer B.Cu) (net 1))
 (segment (start 107.92 77) (end 107.92 84) (width 0.25) (layer B.Cu) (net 1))
 (via (at 137.08 90) (size 0.6) (drill 0.4) (layers F.Cu B.Cu) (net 9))
 (segment (start 137.08 90) (end 137.08 97) (width 0.25) (layer B.Cu) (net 9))
 (segment (start 176.08 90) (end 177 90) (width 0.25) (layer F.Cu) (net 9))
 (segment (start 177 90) (end 178.25 90) (width 0.25) (layer B.Cu) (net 9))
 (via (at 177 90) (size 0.6) (drill 0.4) (layers F.Cu B.Cu) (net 9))
 (via (at 176.08 90) (size 0.6) (drill 0.4) (layers F.Cu B.Cu) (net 9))
 (via (at 157.08 90) (size 0.6) (drill 0.4) (layers F.Cu B.Cu) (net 9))
 (segment (start 118 90) (end 137.08 90) (width 0.25) (layer F.Cu) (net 9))
 (segment (start 137.08 90) (end 157.08 90) (width 0.25) (layer F.Cu) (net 9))
 (segment (start 157.08 90) (end 176.08 90) (width 0.25) (layer F.Cu) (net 9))
 (via (at 118.08 90) (size 0.6) (drill 0.4) (layers F.Cu B.Cu) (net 9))
 (segment (start 118.08 90) (end 118 90) (width 0.25) (layer F.Cu) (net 9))
 (segment (start 176.08 90) (end 176.08 97) (width 0.25) (layer B.Cu) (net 9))
 (segment (start 157.08 90) (end 157.08 97) (width 0.25) (layer B.Cu) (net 9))
 (segment (start 118.08 90) (end 118.08 97) (width 0.25) (layer B.Cu) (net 9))
 (via (at 113 85.73) (size 0.6) (drill 0.4) (layers F.Cu B.Cu) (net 3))
 (segment (start 113 77) (end 113 85.73) (width 0.25) (layer B.Cu) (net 3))
 (segment (start 113 85.73) (end 113 97) (width 0.25) (layer B.Cu) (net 3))
 (segment (start 101.127 85.73) (end 113 85.73) (width 0.25) (layer F.Cu) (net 3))
 (segment (start 179.75 83) (end 182.683 83) (width 0.25) (layer B.Cu) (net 14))
 (segment (start 182.683 83) (end 182.873 83.19) (width 0.25) (layer B.Cu) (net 14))
 (segment (start 179.75 80) (end 182.477 80) (width 0.25) (layer B.Cu) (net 13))
 (segment (start 182.477 80) (end 183.127 80.65) (width 0.25) (layer B.Cu) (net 13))
 (segment (start 179.75 93) (end 182.523 93) (width 0.25) (layer B.Cu) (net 16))
 (segment (start 182.523 93) (end 182.873 93.35) (width 0.25) (layer B.Cu) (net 16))
 (segment (start 104.25 91) (end 101.317 91) (width 0.25) (layer B.Cu) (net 19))
 (segment (start 101.317 91) (end 101.127 90.81) (width 0.25) (layer B.Cu) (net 19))
 (segment (start 104.25 94) (end 101.523 94) (width 0.25) (layer B.Cu) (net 20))
 (segment (start 101.523 94) (end 100.873 93.35) (width 0.25) (layer B.Cu) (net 20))
 (segment (start 104.25 81) (end 101.477 81) (width 0.25) (layer B.Cu) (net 17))
 (segment (start 101.477 81) (end 101.127 80.65) (width 0.25) (layer B.Cu) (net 17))
 (segment (start 104.25 84) (end 101.683 84) (width 0.25) (layer B.Cu) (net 18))
 (segment (start 101.683 84) (end 100.873 83.19) (width 0.25) (layer B.Cu) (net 18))
 (segment (start 179.75 90) (end 182.317 90) (width 0.25) (layer B.Cu) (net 15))
 (segment (start 182.317 90) (end 183.127 90.81) (width 0.25) (layer B.Cu) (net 15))
 (segment (start 132 77) (end 132 88.27) (width 0.25) (layer B.Cu) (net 12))
 (segment (start 132 88.27) (end 132 97) (width 0.25) (layer B.Cu) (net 12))
 (via (at 132 88.27) (size 0.6) (drill 0.4) (layers F.Cu B.Cu) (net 12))
 (segment (start 132 88.27) (end 100.873 88.27) (width 0.25) (layer F.Cu) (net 12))
 (via (at 152 85.73) (size 0.6) (drill 0.4) (layers F.Cu B.Cu) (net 11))
 (segment (start 152 85.73) (end 183.127 85.73) (width 0.25) (layer F.Cu) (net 11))
 (segment (start 152 77) (end 152 85.73) (width 0.25) (layer B.Cu) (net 11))
 (segment (start 152 85.73) (end 152 97) (width 0.25) (layer B.Cu) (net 11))
 (segment (start 182.873 88.27) (end 171 88.27) (width 0.25) (layer F.Cu) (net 10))
 (via (at 171 88.27) (size 0.6) (drill 0.4) (layers F.Cu B.Cu) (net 10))
 (segment (start 171 77) (end 171 88.27) (width 0.25) (layer B.Cu) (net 10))
 (segment (start 171 88.27) (end 171 97) (width 0.25) (layer B.Cu) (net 10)))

